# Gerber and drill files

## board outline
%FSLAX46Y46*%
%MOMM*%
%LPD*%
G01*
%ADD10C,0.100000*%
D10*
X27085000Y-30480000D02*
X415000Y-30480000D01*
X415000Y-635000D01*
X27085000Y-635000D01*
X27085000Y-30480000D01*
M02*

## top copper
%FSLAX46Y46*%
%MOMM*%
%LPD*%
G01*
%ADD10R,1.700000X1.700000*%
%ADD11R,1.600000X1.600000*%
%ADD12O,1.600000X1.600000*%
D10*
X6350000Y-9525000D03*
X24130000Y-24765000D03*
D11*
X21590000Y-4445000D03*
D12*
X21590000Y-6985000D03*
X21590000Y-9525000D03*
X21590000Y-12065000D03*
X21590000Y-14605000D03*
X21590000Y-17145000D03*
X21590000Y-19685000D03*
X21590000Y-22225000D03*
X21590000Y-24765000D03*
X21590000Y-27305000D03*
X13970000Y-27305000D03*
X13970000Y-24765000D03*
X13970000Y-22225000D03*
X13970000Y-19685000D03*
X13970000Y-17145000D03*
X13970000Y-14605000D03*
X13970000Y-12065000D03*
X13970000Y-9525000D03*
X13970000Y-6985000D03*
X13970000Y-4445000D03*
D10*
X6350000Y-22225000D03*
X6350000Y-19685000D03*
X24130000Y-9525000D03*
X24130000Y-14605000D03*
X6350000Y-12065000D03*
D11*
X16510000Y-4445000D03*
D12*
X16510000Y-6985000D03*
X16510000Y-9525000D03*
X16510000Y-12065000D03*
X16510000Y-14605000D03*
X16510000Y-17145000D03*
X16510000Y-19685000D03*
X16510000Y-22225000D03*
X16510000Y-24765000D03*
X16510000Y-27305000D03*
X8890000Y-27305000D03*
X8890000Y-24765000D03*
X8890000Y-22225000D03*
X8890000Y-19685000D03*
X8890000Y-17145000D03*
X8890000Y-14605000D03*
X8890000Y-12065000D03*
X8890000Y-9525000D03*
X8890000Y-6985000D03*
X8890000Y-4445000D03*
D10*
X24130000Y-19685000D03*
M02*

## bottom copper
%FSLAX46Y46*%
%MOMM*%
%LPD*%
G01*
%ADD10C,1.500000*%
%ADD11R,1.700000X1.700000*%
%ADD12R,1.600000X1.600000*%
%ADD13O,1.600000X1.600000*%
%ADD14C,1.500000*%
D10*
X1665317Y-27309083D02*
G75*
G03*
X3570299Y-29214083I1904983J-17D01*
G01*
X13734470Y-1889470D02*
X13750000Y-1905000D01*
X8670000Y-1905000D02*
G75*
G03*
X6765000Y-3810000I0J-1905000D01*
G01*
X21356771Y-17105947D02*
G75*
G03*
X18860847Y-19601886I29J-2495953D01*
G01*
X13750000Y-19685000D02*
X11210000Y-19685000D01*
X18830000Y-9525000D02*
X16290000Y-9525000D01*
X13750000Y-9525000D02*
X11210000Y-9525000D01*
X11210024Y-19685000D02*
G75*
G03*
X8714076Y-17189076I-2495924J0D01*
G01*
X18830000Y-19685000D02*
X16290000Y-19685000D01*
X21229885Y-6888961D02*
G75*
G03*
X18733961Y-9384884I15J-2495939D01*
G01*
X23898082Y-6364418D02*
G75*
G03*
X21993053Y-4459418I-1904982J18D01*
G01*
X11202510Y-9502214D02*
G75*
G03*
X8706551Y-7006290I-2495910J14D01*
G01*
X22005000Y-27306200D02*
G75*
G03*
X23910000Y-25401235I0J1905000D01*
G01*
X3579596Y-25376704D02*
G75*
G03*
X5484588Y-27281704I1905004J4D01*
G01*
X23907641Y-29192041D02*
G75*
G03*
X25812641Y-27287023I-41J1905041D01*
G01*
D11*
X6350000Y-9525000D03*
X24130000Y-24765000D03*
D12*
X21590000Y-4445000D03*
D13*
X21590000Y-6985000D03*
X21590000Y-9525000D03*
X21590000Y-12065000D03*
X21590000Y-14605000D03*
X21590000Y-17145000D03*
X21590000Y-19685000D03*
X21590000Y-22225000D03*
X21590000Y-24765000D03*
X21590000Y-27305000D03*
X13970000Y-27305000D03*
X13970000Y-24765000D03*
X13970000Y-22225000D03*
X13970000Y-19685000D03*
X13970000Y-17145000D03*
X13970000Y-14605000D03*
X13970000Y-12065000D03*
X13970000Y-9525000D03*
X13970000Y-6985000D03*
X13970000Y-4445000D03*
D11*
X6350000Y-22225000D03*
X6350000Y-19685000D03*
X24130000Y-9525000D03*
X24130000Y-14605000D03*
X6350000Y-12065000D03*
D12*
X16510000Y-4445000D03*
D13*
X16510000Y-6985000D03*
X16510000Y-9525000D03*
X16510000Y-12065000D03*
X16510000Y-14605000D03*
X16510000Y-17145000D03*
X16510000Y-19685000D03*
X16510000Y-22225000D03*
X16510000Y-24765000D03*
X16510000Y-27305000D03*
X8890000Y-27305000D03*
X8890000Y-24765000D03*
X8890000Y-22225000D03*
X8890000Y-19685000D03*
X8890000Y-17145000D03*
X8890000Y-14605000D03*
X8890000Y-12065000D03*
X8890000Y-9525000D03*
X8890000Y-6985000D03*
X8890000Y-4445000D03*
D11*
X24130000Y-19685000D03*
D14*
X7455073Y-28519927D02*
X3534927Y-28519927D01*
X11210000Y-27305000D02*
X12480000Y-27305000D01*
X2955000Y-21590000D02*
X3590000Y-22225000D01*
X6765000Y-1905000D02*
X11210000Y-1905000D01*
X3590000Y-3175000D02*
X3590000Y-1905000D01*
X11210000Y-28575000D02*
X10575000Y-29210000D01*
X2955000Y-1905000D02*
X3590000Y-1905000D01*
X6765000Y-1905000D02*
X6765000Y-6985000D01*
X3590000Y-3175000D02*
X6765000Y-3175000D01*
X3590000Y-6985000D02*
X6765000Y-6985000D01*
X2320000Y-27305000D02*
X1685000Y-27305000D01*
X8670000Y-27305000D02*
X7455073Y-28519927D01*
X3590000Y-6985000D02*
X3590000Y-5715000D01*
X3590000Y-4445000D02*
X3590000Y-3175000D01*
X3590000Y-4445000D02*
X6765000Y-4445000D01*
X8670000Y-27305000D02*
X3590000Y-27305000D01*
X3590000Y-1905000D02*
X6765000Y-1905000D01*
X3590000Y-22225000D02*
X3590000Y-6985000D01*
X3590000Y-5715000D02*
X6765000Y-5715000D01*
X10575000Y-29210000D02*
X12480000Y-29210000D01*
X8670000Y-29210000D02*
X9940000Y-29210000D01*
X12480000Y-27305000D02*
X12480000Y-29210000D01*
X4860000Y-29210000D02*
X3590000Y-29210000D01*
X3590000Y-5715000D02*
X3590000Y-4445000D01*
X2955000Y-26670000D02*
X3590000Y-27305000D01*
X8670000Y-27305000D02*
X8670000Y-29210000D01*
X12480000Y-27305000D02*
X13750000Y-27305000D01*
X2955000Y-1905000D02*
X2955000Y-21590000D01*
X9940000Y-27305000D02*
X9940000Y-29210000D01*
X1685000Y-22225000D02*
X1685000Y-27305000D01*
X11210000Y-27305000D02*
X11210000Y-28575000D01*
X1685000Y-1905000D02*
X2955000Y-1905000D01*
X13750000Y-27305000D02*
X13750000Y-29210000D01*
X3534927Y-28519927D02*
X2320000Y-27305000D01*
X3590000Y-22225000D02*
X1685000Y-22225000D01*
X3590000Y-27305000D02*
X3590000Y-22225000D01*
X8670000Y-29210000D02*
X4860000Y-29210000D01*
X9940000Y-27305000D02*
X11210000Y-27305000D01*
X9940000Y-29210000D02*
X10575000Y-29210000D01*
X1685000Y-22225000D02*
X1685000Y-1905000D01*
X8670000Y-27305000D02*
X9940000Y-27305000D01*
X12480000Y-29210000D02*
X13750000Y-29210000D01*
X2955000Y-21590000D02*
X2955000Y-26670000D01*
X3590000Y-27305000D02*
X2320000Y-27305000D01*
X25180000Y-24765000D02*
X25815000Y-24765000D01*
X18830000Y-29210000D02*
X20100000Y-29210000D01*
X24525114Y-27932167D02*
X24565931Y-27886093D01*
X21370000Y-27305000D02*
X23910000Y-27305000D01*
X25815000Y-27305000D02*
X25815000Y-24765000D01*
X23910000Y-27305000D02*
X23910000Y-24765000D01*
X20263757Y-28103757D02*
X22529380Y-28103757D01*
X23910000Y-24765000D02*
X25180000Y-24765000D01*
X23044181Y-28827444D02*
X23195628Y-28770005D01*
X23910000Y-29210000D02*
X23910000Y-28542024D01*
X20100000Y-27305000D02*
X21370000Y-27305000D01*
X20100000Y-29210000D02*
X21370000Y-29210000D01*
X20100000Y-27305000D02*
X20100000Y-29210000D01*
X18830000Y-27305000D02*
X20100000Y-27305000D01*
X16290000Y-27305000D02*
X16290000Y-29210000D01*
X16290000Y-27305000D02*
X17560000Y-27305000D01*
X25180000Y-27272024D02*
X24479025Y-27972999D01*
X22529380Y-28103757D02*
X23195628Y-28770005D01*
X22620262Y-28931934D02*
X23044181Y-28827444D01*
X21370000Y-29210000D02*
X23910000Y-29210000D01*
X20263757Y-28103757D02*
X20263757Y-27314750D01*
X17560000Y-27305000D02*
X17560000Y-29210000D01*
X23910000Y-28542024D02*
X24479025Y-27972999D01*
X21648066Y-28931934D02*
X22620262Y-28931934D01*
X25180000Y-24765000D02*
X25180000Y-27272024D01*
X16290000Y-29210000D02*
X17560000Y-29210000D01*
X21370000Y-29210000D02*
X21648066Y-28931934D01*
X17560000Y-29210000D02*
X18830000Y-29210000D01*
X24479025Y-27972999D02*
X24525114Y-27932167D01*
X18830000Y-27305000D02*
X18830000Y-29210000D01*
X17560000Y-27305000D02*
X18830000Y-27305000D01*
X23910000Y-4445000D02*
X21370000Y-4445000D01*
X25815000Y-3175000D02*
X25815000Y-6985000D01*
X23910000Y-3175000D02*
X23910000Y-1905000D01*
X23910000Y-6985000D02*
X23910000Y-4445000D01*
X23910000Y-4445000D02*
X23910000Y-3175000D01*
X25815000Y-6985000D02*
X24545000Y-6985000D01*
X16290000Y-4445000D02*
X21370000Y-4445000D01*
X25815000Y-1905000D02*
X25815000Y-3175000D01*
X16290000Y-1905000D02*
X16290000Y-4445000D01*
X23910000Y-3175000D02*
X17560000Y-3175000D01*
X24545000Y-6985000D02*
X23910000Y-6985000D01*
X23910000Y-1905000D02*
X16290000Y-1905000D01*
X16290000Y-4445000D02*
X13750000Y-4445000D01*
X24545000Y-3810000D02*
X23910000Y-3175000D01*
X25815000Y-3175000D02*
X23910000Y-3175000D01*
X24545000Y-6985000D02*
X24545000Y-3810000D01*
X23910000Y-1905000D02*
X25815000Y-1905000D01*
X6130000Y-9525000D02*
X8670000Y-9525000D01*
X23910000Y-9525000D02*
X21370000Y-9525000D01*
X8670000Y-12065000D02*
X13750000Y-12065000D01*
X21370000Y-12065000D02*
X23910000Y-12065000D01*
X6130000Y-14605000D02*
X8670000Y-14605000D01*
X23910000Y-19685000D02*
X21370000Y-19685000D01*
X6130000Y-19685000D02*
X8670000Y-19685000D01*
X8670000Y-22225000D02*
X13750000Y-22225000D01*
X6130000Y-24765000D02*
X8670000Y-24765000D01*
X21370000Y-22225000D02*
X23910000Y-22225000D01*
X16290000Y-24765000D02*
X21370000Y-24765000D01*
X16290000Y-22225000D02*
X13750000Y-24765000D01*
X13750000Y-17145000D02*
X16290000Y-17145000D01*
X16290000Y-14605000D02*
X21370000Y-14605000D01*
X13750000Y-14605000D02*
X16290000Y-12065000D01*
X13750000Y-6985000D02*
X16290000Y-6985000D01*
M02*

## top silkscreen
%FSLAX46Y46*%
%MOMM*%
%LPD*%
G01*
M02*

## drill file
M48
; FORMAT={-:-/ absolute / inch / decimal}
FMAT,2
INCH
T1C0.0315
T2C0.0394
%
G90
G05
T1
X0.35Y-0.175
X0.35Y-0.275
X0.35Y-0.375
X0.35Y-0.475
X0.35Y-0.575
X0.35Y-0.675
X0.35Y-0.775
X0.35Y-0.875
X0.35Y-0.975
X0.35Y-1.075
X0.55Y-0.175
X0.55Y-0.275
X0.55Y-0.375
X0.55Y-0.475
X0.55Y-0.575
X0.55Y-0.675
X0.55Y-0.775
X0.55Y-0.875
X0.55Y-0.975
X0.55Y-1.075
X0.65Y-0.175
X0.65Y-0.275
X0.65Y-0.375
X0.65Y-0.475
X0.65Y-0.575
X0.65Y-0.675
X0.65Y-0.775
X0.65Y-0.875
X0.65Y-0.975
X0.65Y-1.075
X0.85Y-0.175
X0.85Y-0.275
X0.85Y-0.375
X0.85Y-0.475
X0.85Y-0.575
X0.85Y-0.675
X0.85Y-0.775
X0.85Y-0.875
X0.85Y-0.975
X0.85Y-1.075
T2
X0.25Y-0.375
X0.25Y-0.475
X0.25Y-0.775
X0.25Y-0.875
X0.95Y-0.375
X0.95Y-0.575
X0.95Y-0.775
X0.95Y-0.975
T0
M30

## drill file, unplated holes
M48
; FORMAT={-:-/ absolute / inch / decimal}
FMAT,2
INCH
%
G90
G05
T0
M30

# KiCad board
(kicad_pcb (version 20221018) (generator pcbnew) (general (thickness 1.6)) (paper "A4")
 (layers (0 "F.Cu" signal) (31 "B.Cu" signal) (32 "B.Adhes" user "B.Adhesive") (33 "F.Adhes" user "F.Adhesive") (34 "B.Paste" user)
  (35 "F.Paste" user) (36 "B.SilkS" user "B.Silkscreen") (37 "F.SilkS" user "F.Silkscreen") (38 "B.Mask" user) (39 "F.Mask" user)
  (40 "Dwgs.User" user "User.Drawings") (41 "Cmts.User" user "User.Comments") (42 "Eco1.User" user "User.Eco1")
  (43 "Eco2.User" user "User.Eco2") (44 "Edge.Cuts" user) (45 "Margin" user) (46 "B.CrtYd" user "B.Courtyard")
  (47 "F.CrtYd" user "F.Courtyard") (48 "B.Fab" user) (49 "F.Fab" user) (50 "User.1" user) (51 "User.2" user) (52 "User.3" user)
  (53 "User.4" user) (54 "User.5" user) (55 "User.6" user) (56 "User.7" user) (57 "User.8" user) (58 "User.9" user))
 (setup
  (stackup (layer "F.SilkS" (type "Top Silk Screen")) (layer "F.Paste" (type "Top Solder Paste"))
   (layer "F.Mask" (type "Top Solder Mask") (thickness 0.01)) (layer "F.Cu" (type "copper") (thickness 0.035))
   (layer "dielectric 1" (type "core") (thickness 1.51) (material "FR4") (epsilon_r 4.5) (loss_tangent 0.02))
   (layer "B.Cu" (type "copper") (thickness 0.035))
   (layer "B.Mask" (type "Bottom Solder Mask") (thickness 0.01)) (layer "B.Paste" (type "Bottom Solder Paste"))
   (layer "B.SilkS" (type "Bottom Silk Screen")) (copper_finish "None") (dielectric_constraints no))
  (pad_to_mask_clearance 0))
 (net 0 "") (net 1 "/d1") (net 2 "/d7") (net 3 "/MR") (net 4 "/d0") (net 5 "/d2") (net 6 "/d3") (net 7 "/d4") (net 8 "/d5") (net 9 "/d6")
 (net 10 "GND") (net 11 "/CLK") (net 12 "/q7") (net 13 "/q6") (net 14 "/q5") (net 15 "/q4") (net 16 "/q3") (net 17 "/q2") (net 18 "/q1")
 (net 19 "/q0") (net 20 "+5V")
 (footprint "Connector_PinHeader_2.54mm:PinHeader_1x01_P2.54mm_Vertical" (layer "B.Cu") (at 6.35 9.525 180)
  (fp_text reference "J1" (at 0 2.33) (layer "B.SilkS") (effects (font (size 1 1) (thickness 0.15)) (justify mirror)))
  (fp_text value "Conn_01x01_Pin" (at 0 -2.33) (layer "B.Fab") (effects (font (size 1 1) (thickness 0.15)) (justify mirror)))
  (pad "1" thru_hole rect (at 0 0 180) (size 1.7 1.7) (drill 1) (layers "*.Cu" "*.Mask") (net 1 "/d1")))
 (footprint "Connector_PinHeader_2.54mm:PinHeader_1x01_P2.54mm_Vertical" (layer "B.Cu") (at 24.13 24.765 180)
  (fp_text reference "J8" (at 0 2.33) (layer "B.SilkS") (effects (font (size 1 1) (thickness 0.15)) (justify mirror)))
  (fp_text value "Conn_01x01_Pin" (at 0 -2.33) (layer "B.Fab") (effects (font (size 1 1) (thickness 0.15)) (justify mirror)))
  (pad "1" thru_hole rect (at 0 0 180) (size 1.7 1.7) (drill 1) (layers "*.Cu" "*.Mask") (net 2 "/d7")))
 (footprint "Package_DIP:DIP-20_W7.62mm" (layer "B.Cu") (at 21.59 4.445 180)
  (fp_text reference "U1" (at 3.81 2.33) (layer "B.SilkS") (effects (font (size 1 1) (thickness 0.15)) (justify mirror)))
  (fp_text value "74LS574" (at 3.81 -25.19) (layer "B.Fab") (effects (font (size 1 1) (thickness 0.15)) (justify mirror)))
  (pad "1" thru_hole rect (at 0 0 180) (size 1.6 1.6) (drill 0.8) (layers "*.Cu" "*.Mask") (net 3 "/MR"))
  (pad "2" thru_hole oval (at 0 -2.54 180) (size 1.6 1.6) (drill 0.8) (layers "*.Cu" "*.Mask") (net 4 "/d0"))
  (pad "3" thru_hole oval (at 0 -5.08 180) (size 1.6 1.6) (drill 0.8) (layers "*.Cu" "*.Mask") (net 1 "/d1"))
  (pad "4" thru_hole oval (at 0 -7.62 180) (size 1.6 1.6) (drill 0.8) (layers "*.Cu" "*.Mask") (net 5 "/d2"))
  (pad "5" thru_hole oval (at 0 -10.16 180) (size 1.6 1.6) (drill 0.8) (layers "*.Cu" "*.Mask") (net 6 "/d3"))
  (pad "6" thru_hole oval (at 0 -12.7 180) (size 1.6 1.6) (drill 0.8) (layers "*.Cu" "*.Mask") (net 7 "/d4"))
  (pad "7" thru_hole oval (at 0 -15.24 180) (size 1.6 1.6) (drill 0.8) (layers "*.Cu" "*.Mask") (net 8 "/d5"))
  (pad "8" thru_hole oval (at 0 -17.78 180) (size 1.6 1.6) (drill 0.8) (layers "*.Cu" "*.Mask") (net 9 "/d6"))
  (pad "9" thru_hole oval (at 0 -20.32 180) (size 1.6 1.6) (drill 0.8) (layers "*.Cu" "*.Mask") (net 2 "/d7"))
  (pad "10" thru_hole oval (at 0 -22.86 180) (size 1.6 1.6) (drill 0.8) (layers "*.Cu" "*.Mask") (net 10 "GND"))
  (pad "11" thru_hole oval (at 7.62 -22.86 180) (size 1.6 1.6) (drill 0.8) (layers "*.Cu" "*.Mask") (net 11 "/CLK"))
  (pad "12" thru_hole oval (at 7.62 -20.32 180) (size 1.6 1.6) (drill 0.8) (layers "*.Cu" "*.Mask") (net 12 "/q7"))
  (pad "13" thru_hole oval (at 7.62 -17.78 180) (size 1.6 1.6) (drill 0.8) (layers "*.Cu" "*.Mask") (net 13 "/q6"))
  (pad "14" thru_hole oval (at 7.62 -15.24 180) (size 1.6 1.6) (drill 0.8) (layers "*.Cu" "*.Mask") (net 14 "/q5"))
  (pad "15" thru_hole oval (at 7.62 -12.7 180) (size 1.6 1.6) (drill 0.8) (layers "*.Cu" "*.Mask") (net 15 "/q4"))
  (pad "16" thru_hole oval (at 7.62 -10.16 180) (size 1.6 1.6) (drill 0.8) (layers "*.Cu" "*.Mask") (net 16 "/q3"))
  (pad "17" thru_hole oval (at 7.62 -7.62 180) (size 1.6 1.6) (drill 0.8) (layers "*.Cu" "*.Mask") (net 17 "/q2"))
  (pad "18" thru_hole oval (at 7.62 -5.08 180) (size 1.6 1.6) (drill 0.8) (layers "*.Cu" "*.Mask") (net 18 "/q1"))
  (pad "19" thru_hole oval (at 7.62 -2.54 180) (size 1.6 1.6) (drill 0.8) (layers "*.Cu" "*.Mask") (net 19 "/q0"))
  (pad "20" thru_hole oval (at 7.62 0 180) (size 1.6 1.6) (drill 0.8) (layers "*.Cu" "*.Mask") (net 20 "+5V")))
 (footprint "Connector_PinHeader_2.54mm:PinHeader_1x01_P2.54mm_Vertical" (layer "B.Cu") (at 6.35 22.225 180)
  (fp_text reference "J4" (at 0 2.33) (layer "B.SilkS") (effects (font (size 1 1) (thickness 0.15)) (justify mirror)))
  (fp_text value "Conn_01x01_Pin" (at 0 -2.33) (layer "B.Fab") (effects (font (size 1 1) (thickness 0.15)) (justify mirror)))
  (pad "1" thru_hole rect (at 0 0 180) (size 1.7 1.7) (drill 1) (layers "*.Cu" "*.Mask") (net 2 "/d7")))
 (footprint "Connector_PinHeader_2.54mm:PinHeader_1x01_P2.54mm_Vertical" (layer "B.Cu") (at 6.35 19.685 180)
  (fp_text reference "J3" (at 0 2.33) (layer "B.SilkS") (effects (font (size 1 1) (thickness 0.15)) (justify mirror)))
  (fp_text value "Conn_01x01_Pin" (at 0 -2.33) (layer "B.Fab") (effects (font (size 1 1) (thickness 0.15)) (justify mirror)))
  (pad "1" thru_hole rect (at 0 0 180) (size 1.7 1.7) (drill 1) (layers "*.Cu" "*.Mask") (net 8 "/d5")))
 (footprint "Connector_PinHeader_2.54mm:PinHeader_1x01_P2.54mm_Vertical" (layer "B.Cu") (at 24.13 9.525 180)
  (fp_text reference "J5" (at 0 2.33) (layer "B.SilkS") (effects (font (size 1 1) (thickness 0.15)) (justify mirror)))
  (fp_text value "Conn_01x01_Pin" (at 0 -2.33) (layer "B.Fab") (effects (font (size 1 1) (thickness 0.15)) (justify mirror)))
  (pad "1" thru_hole rect (at 0 0 180) (size 1.7 1.7) (drill 1) (layers "*.Cu" "*.Mask") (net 1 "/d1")))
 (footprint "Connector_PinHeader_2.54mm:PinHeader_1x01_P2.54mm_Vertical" (layer "B.Cu") (at 24.13 14.605 180)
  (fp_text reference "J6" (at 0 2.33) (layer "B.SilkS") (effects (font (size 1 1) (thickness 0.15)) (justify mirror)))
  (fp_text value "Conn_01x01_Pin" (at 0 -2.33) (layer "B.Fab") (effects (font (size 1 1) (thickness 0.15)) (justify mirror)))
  (pad "1" thru_hole rect (at 0 0 180) (size 1.7 1.7) (drill 1) (layers "*.Cu" "*.Mask") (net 6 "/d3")))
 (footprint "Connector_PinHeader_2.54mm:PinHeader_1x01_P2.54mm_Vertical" (layer "B.Cu") (at 6.35 12.065 180)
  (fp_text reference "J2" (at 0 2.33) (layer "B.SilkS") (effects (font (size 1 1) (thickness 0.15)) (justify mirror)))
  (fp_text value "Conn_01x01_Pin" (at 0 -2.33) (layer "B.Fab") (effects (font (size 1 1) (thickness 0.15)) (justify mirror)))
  (pad "1" thru_hole rect (at 0 0 180) (size 1.7 1.7) (drill 1) (layers "*.Cu" "*.Mask") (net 6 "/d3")))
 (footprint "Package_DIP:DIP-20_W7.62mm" (layer "B.Cu") (at 16.51 4.445 180)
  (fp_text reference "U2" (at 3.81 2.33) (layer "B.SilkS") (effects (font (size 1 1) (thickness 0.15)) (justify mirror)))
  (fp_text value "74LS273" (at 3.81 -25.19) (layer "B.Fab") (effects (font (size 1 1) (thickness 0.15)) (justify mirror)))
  (pad "1" thru_hole rect (at 0 0 180) (size 1.6 1.6) (drill 0.8) (layers "*.Cu" "*.Mask") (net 20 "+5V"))
  (pad "2" thru_hole oval (at 0 -2.54 180) (size 1.6 1.6) (drill 0.8) (layers "*.Cu" "*.Mask") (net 19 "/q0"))
  (pad "3" thru_hole oval (at 0 -5.08 180) (size 1.6 1.6) (drill 0.8) (layers "*.Cu" "*.Mask") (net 4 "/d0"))
  (pad "4" thru_hole oval (at 0 -7.62 180) (size 1.6 1.6) (drill 0.8) (layers "*.Cu" "*.Mask") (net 5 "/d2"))
  (pad "5" thru_hole oval (at 0 -10.16 180) (size 1.6 1.6) (drill 0.8) (layers "*.Cu" "*.Mask") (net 17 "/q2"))
  (pad "6" thru_hole oval (at 0 -12.7 180) (size 1.6 1.6) (drill 0.8) (layers "*.Cu" "*.Mask") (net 15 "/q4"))
  (pad "7" thru_hole oval (at 0 -15.24 180) (size 1.6 1.6) (drill 0.8) (layers "*.Cu" "*.Mask") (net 7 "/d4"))
  (pad "8" thru_hole oval (at 0 -17.78 180) (size 1.6 1.6) (drill 0.8) (layers "*.Cu" "*.Mask") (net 9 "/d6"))
  (pad "9" thru_hole oval (at 0 -20.32 180) (size 1.6 1.6) (drill 0.8) (layers "*.Cu" "*.Mask") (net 13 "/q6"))
  (pad "10" thru_hole oval (at 0 -22.86 180) (size 1.6 1.6) (drill 0.8) (layers "*.Cu" "*.Mask") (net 10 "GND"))
  (pad "11" thru_hole oval (at 7.62 -22.86 180) (size 1.6 1.6) (drill 0.8) (layers "*.Cu" "*.Mask") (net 11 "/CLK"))
  (pad "12" thru_hole oval (at 7.62 -20.32 180) (size 1.6 1.6) (drill 0.8) (layers "*.Cu" "*.Mask") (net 12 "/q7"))
  (pad "13" thru_hole oval (at 7.62 -17.78 180) (size 1.6 1.6) (drill 0.8) (layers "*.Cu" "*.Mask") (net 2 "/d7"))
  (pad "14" thru_hole oval (at 7.62 -15.24 180) (size 1.6 1.6) (drill 0.8) (layers "*.Cu" "*.Mask") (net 8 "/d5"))
  (pad "15" thru_hole oval (at 7.62 -12.7 180) (size 1.6 1.6) (drill 0.8) (layers "*.Cu" "*.Mask") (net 14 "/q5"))
  (pad "16" thru_hole oval (at 7.62 -10.16 180) (size 1.6 1.6) (drill 0.8) (layers "*.Cu" "*.Mask") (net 16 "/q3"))
  (pad "17" thru_hole oval (at 7.62 -7.62 180) (size 1.6 1.6) (drill 0.8) (layers "*.Cu" "*.Mask") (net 6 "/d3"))
  (pad "18" thru_hole oval (at 7.62 -5.08 180) (size 1.6 1.6) (drill 0.8) (layers "*.Cu" "*.Mask") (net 1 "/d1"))
  (pad "19" thru_hole oval (at 7.62 -2.54 180) (size 1.6 1.6) (drill 0.8) (layers "*.Cu" "*.Mask") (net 18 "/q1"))
  (pad "20" thru_hole oval (at 7.62 0 180) (size 1.6 1.6) (drill 0.8) (layers "*.Cu" "*.Mask") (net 20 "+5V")))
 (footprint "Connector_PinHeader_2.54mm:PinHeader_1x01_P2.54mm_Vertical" (layer "B.Cu") (at 24.13 19.685 180)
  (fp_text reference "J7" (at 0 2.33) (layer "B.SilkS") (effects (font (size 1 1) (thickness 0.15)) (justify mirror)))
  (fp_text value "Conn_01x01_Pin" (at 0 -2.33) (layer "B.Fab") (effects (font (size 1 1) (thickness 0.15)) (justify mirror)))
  (pad "1" thru_hole rect (at 0 0 180) (size 1.7 1.7) (drill 1) (layers "*.Cu" "*.Mask") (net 8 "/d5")))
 (gr_arc (start 3.570299 29.214083) (mid 2.223267 28.65612) (end 1.665299 27.309083) (stroke (width 1.5) (type default)) (layer "B.Cu"))
 (gr_line (start 13.73447 1.88947) (end 13.75 1.905) (stroke (width 1.5) (type default)) (layer "B.Cu"))
 (gr_arc (start 6.765 3.81) (mid 7.322962 2.462962) (end 8.67 1.905) (stroke (width 1.5) (type default)) (layer "B.Cu"))
 (gr_arc (start 18.860847 19.601886) (mid 19.591889 17.837) (end 21.356771 17.105962) (stroke (width 1.5) (type default)) (layer "B.Cu"))
 (gr_line (start 13.75 19.685) (end 11.21 19.685) (stroke (width 1.5) (type default)) (layer "B.Cu"))
 (gr_line (start 18.83 9.525) (end 16.29 9.525) (stroke (width 1.5) (type default)) (layer "B.Cu"))
 (gr_line (start 13.75 9.525) (end 11.21 9.525) (stroke (width 1.5) (type default)) (layer "B.Cu"))
 (gr_arc (start 8.714076 17.189076) (mid 10.478976 17.920107) (end 11.21 19.685) (stroke (width 1.5) (type default)) (layer "B.Cu"))
 (gr_line (start 18.83 19.685) (end 16.29 19.685) (stroke (width 1.5) (type default)) (layer "B.Cu"))
 (gr_arc (start 18.733961 9.384884) (mid 19.465005 7.620004) (end 21.229885 6.88896) (stroke (width 1.5) (type default)) (layer "B.Cu"))
 (gr_arc (start 21.993053 4.459418) (mid 23.340115 5.017364) (end 23.898053 6.364418) (stroke (width 1.5) (type default)) (layer "B.Cu"))
 (gr_arc (start 8.706551 7.00629) (mid 10.471463 7.737313) (end 11.202475 9.502214) (stroke (width 1.5) (type default)) (layer "B.Cu"))
 (gr_arc (start 23.91 25.401235) (mid 23.352026 26.748251) (end 22.005 27.306235) (stroke (width 1.5) (type default)) (layer "B.Cu"))
 (gr_arc (start 5.484588 27.281704) (mid 4.137556 26.723738) (end 3.579588 25.376704) (stroke (width 1.5) (type default)) (layer "B.Cu"))
 (gr_arc (start 25.812641 27.287023) (mid 25.254674 28.634061) (end 23.907641 29.192023) (stroke (width 1.5) (type default)) (layer "B.Cu"))
 (gr_rect (start 27.085 30.48) (end 0.415 0.635) (stroke (width 0.1) (type default)) (fill none) (layer "Edge.Cuts"))
 (segment (start 7.455073 28.519927) (end 3.534927 28.519927) (width 1.5) (layer "B.Cu") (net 11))
 (segment (start 11.21 27.305) (end 12.48 27.305) (width 1.5) (layer "B.Cu") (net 11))
 (segment (start 2.955 21.59) (end 3.59 22.225) (width 1.5) (layer "B.Cu") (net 11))
 (segment (start 6.765 1.905) (end 11.21 1.905) (width 1.5) (layer "B.Cu") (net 11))
 (segment (start 3.59 3.175) (end 3.59 1.905) (width 1.5) (layer "B.Cu") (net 11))
 (segment (start 25.18 24.765) (end 25.815 24.765) (width 1.5) (layer "B.Cu") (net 11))
 (segment (start 11.21 28.575) (end 10.575 29.21) (width 1.5) (layer "B.Cu") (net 11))
 (segment (start 2.955 1.905) (end 3.59 1.905) (width 1.5) (layer "B.Cu") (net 11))
 (segment (start 6.765 1.905) (end 6.765 6.985) (width 1.5) (layer "B.Cu") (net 11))
 (segment (start 18.83 29.21) (end 20.1 29.21) (width 1.5) (layer "B.Cu") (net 11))
 (segment (start 3.59 3.175) (end 6.765 3.175) (width 1.5) (layer "B.Cu") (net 11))
 (segment (start 3.59 6.985) (end 6.765 6.985) (width 1.5) (layer "B.Cu") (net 11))
 (segment (start 2.32 27.305) (end 1.685 27.305) (width 1.5) (layer "B.Cu") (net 11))
 (segment (start 8.67 27.305) (end 7.455073 28.519927) (width 1.5) (layer "B.Cu") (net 11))
 (segment (start 24.525114 27.932167) (end 24.565931 27.886093) (width 1.5) (layer "B.Cu") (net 11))
 (segment (start 21.37 27.305) (end 23.91 27.305) (width 1.5) (layer "B.Cu") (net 11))
 (segment (start 25.815 27.305) (end 25.815 24.765) (width 1.5) (layer "B.Cu") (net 11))
 (segment (start 23.91 27.305) (end 23.91 24.765) (width 1.5) (layer "B.Cu") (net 11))
 (segment (start 20.263757 28.103757) (end 22.52938 28.103757) (width 1.5) (layer "B.Cu") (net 11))
 (segment (start 3.59 6.985) (end 3.59 5.715) (width 1.5) (layer "B.Cu") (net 11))
 (segment (start 23.91 24.765) (end 25.18 24.765) (width 1.5) (layer "B.Cu") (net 11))
 (segment (start 23.044181 28.827444) (end 23.195628 28.770005) (width 1.5) (layer "B.Cu") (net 11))
 (segment (start 23.91 29.21) (end 23.91 28.542024) (width 1.5) (layer "B.Cu") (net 11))
 (segment (start 3.59 4.445) (end 3.59 3.175) (width 1.5) (layer "B.Cu") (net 11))
 (segment (start 3.59 4.445) (end 6.765 4.445) (width 1.5) (layer "B.Cu") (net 11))
 (segment (start 8.67 27.305) (end 3.59 27.305) (width 1.5) (layer "B.Cu") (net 11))
 (segment (start 3.59 1.905) (end 6.765 1.905) (width 1.5) (layer "B.Cu") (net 11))
 (segment (start 20.1 27.305) (end 21.37 27.305) (width 1.5) (layer "B.Cu") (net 11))
 (segment (start 20.1 29.21) (end 21.37 29.21) (width 1.5) (layer "B.Cu") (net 11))
 (segment (start 3.59 22.225) (end 3.59 6.985) (width 1.5) (layer "B.Cu") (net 11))
 (segment (start 20.1 27.305) (end 20.1 29.21) (width 1.5) (layer "B.Cu") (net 11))
 (segment (start 3.59 5.715) (end 6.765 5.715) (width 1.5) (layer "B.Cu") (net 11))
 (segment (start 10.575 29.21) (end 12.48 29.21) (width 1.5) (layer "B.Cu") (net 11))
 (segment (start 8.67 29.21) (end 9.94 29.21) (width 1.5) (layer "B.Cu") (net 11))
 (segment (start 12.48 27.305) (end 12.48 29.21) (width 1.5) (layer "B.Cu") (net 11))
 (segment (start 4.86 29.21) (end 3.59 29.21) (width 1.5) (layer "B.Cu") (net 11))
 (segment (start 3.59 5.715) (end 3.59 4.445) (width 1.5) (layer "B.Cu") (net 11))
 (segment (start 2.955 26.67) (end 3.59 27.305) (width 1.5) (layer "B.Cu") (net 11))
 (segment (start 18.83 27.305) (end 20.1 27.305) (width 1.5) (layer "B.Cu") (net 11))
 (segment (start 16.29 27.305) (end 16.29 29.21) (width 1.5) (layer "B.Cu") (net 11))
 (segment (start 8.67 27.305) (end 8.67 29.21) (width 1.5) (layer "B.Cu") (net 11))
 (segment (start 12.48 27.305) (end 13.75 27.305) (width 1.5) (layer "B.Cu") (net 11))
 (segment (start 2.955 1.905) (end 2.955 21.59) (width 1.5) (layer "B.Cu") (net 11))
 (segment (start 9.94 27.305) (end 9.94 29.21) (width 1.5) (layer "B.Cu") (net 11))
 (segment (start 16.29 27.305) (end 17.56 27.305) (width 1.5) (layer "B.Cu") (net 11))
 (segment (start 1.685 22.225) (end 1.685 27.305) (width 1.5) (layer "B.Cu") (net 11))
 (segment (start 11.21 27.305) (end 11.21 28.575) (width 1.5) (layer "B.Cu") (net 11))
 (segment (start 25.18 27.272024) (end 24.479025 27.972999) (width 1.5) (layer "B.Cu") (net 11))
 (segment (start 1.685 1.905) (end 2.955 1.905) (width 1.5) (layer "B.Cu") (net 11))
 (segment (start 22.52938 28.103757) (end 23.195628 28.770005) (width 1.5) (layer "B.Cu") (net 11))
 (segment (start 13.75 27.305) (end 13.75 29.21) (width 1.5) (layer "B.Cu") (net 11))
 (segment (start 22.620262 28.931934) (end 23.044181 28.827444) (width 1.5) (layer "B.Cu") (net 11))
 (segment (start 21.37 29.21) (end 23.91 29.21) (width 1.5) (layer "B.Cu") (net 11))
 (segment (start 20.263757 28.103757) (end 20.263757 27.31475) (width 1.5) (layer "B.Cu") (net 11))
 (segment (start 17.56 27.305) (end 17.56 29.21) (width 1.5) (layer "B.Cu") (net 11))
 (segment (start 3.534927 28.519927) (end 2.32 27.305) (width 1.5) (layer "B.Cu") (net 11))
 (segment (start 3.59 22.225) (end 1.685 22.225) (width 1.5) (layer "B.Cu") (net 11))
 (segment (start 23.91 28.542024) (end 24.479025 27.972999) (width 1.5) (layer "B.Cu") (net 11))
 (segment (start 3.59 27.305) (end 3.59 22.225) (width 1.5) (layer "B.Cu") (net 11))
 (segment (start 8.67 29.21) (end 4.86 29.21) (width 1.5) (layer "B.Cu") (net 11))
 (segment (start 21.648066 28.931934) (end 22.620262 28.931934) (width 1.5) (layer "B.Cu") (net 11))
 (segment (start 25.18 24.765) (end 25.18 27.272024) (width 1.5) (layer "B.Cu") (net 11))
 (segment (start 16.29 29.21) (end 17.56 29.21) (width 1.5) (layer "B.Cu") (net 11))
 (segment (start 21.37 29.21) (end 21.648066 28.931934) (width 1.5) (layer "B.Cu") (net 11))
 (segment (start 17.56 29.21) (end 18.83 29.21) (width 1.5) (layer "B.Cu") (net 11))
 (segment (start 9.94 27.305) (end 11.21 27.305) (width 1.5) (layer "B.Cu") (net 11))
 (segment (start 9.94 29.21) (end 10.575 29.21) (width 1.5) (layer "B.Cu") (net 11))
 (segment (start 1.685 22.225) (end 1.685 1.905) (width 1.5) (layer "B.Cu") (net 11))
 (segment (start 8.67 27.305) (end 9.94 27.305) (width 1.5) (layer "B.Cu") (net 11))
 (segment (start 24.479025 27.972999) (end 24.525114 27.932167) (width 1.5) (layer "B.Cu") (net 11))
 (segment (start 18.83 27.305) (end 18.83 29.21) (width 1.5) (layer "B.Cu") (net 11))
 (segment (start 17.56 27.305) (end 18.83 27.305) (width 1.5) (layer "B.Cu") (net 11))
 (segment (start 12.48 29.21) (end 13.75 29.21) (width 1.5) (layer "B.Cu") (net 11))
 (segment (start 2.955 21.59) (end 2.955 26.67) (width 1.5) (layer "B.Cu") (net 11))
 (segment (start 3.59 27.305) (end 2.32 27.305) (width 1.5) (layer "B.Cu") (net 11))
 (segment (start 23.91 4.445) (end 21.37 4.445) (width 1.5) (layer "B.Cu") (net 20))
 (segment (start 25.815 3.175) (end 25.815 6.985) (width 1.5) (layer "B.Cu") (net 20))
 (segment (start 23.91 3.175) (end 23.91 1.905) (width 1.5) (layer "B.Cu") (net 20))
 (segment (start 23.91 6.985) (end 23.91 4.445) (width 1.5) (layer "B.Cu") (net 20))
 (segment (start 23.91 4.445) (end 23.91 3.175) (width 1.5) (layer "B.Cu") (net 20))
 (segment (start 25.815 6.985) (end 24.545 6.985) (width 1.5) (layer "B.Cu") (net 20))
 (segment (start 16.29 4.445) (end 21.37 4.445) (width 1.5) (layer "B.Cu") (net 20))
 (segment (start 25.815 1.905) (end 25.815 3.175) (width 1.5) (layer "B.Cu") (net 20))
 (segment (start 16.29 1.905) (end 16.29 4.445) (width 1.5) (layer "B.Cu") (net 20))
 (segment (start 23.91 3.175) (end 17.56 3.175) (width 1.5) (layer "B.Cu") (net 20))
 (segment (start 24.545 6.985) (end 23.91 6.985) (width 1.5) (layer "B.Cu") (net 20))
 (segment (start 23.91 1.905) (end 16.29 1.905) (width 1.5) (layer "B.Cu") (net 20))
 (segment (start 16.29 4.445) (end 13.75 4.445) (width 1.5) (layer "B.Cu") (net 20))
 (segment (start 24.545 3.81) (end 23.91 3.175) (width 1.5) (layer "B.Cu") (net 20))
 (segment (start 25.815 3.175) (end 23.91 3.175) (width 1.5) (layer "B.Cu") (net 20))
 (segment (start 24.545 6.985) (end 24.545 3.81) (width 1.5) (layer "B.Cu") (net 20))
 (segment (start 23.91 1.905) (end 25.815 1.905) (width 1.5) (layer "B.Cu") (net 20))
 (segment (start 6.13 9.525) (end 8.67 9.525) (width 1.5) (layer "B.Cu") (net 1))
 (segment (start 23.91 9.525) (end 21.37 9.525) (width 1.5) (layer "B.Cu") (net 1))
 (segment (start 21.37 12.065) (end 23.91 12.065) (width 1.5) (layer "B.Cu") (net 5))
 (segment (start 8.67 12.065) (end 13.75 12.065) (width 1.5) (layer "B.Cu") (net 5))
 (segment (start 23.91 19.685) (end 21.37 19.685) (width 1.5) (layer "B.Cu") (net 8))
 (segment (start 6.13 19.685) (end 8.67 19.685) (width 1.5) (layer "B.Cu") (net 8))
 (segment (start 8.67 22.225) (end 13.75 22.225) (width 1.5) (layer "B.Cu") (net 9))
 (segment (start 21.37 22.225) (end 23.91 22.225) (width 1.5) (layer "B.Cu") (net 9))
 (segment (start 6.13 24.765) (end 8.67 24.765) (width 1.5) (layer "B.Cu") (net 12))
 (segment (start 16.29 24.765) (end 21.37 24.765) (width 1.5) (layer "B.Cu") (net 12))
 (segment (start 16.29 22.225) (end 13.75 24.765) (width 1.5) (layer "B.Cu") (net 13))
 (segment (start 13.75 17.145) (end 16.29 17.145) (width 1.5) (layer "B.Cu") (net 15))
 (segment (start 6.13 14.605) (end 8.67 14.605) (width 1.5) (layer "B.Cu") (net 16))
 (segment (start 16.29 14.605) (end 21.37 14.605) (width 1.5) (layer "B.Cu") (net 16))
 (segment (start 13.75 14.605) (end 16.29 12.065) (width 1.5) (layer "B.Cu") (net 17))
 (segment (start 13.75 6.985) (end 16.29 6.985) (width 1.5) (layer "B.Cu") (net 19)))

